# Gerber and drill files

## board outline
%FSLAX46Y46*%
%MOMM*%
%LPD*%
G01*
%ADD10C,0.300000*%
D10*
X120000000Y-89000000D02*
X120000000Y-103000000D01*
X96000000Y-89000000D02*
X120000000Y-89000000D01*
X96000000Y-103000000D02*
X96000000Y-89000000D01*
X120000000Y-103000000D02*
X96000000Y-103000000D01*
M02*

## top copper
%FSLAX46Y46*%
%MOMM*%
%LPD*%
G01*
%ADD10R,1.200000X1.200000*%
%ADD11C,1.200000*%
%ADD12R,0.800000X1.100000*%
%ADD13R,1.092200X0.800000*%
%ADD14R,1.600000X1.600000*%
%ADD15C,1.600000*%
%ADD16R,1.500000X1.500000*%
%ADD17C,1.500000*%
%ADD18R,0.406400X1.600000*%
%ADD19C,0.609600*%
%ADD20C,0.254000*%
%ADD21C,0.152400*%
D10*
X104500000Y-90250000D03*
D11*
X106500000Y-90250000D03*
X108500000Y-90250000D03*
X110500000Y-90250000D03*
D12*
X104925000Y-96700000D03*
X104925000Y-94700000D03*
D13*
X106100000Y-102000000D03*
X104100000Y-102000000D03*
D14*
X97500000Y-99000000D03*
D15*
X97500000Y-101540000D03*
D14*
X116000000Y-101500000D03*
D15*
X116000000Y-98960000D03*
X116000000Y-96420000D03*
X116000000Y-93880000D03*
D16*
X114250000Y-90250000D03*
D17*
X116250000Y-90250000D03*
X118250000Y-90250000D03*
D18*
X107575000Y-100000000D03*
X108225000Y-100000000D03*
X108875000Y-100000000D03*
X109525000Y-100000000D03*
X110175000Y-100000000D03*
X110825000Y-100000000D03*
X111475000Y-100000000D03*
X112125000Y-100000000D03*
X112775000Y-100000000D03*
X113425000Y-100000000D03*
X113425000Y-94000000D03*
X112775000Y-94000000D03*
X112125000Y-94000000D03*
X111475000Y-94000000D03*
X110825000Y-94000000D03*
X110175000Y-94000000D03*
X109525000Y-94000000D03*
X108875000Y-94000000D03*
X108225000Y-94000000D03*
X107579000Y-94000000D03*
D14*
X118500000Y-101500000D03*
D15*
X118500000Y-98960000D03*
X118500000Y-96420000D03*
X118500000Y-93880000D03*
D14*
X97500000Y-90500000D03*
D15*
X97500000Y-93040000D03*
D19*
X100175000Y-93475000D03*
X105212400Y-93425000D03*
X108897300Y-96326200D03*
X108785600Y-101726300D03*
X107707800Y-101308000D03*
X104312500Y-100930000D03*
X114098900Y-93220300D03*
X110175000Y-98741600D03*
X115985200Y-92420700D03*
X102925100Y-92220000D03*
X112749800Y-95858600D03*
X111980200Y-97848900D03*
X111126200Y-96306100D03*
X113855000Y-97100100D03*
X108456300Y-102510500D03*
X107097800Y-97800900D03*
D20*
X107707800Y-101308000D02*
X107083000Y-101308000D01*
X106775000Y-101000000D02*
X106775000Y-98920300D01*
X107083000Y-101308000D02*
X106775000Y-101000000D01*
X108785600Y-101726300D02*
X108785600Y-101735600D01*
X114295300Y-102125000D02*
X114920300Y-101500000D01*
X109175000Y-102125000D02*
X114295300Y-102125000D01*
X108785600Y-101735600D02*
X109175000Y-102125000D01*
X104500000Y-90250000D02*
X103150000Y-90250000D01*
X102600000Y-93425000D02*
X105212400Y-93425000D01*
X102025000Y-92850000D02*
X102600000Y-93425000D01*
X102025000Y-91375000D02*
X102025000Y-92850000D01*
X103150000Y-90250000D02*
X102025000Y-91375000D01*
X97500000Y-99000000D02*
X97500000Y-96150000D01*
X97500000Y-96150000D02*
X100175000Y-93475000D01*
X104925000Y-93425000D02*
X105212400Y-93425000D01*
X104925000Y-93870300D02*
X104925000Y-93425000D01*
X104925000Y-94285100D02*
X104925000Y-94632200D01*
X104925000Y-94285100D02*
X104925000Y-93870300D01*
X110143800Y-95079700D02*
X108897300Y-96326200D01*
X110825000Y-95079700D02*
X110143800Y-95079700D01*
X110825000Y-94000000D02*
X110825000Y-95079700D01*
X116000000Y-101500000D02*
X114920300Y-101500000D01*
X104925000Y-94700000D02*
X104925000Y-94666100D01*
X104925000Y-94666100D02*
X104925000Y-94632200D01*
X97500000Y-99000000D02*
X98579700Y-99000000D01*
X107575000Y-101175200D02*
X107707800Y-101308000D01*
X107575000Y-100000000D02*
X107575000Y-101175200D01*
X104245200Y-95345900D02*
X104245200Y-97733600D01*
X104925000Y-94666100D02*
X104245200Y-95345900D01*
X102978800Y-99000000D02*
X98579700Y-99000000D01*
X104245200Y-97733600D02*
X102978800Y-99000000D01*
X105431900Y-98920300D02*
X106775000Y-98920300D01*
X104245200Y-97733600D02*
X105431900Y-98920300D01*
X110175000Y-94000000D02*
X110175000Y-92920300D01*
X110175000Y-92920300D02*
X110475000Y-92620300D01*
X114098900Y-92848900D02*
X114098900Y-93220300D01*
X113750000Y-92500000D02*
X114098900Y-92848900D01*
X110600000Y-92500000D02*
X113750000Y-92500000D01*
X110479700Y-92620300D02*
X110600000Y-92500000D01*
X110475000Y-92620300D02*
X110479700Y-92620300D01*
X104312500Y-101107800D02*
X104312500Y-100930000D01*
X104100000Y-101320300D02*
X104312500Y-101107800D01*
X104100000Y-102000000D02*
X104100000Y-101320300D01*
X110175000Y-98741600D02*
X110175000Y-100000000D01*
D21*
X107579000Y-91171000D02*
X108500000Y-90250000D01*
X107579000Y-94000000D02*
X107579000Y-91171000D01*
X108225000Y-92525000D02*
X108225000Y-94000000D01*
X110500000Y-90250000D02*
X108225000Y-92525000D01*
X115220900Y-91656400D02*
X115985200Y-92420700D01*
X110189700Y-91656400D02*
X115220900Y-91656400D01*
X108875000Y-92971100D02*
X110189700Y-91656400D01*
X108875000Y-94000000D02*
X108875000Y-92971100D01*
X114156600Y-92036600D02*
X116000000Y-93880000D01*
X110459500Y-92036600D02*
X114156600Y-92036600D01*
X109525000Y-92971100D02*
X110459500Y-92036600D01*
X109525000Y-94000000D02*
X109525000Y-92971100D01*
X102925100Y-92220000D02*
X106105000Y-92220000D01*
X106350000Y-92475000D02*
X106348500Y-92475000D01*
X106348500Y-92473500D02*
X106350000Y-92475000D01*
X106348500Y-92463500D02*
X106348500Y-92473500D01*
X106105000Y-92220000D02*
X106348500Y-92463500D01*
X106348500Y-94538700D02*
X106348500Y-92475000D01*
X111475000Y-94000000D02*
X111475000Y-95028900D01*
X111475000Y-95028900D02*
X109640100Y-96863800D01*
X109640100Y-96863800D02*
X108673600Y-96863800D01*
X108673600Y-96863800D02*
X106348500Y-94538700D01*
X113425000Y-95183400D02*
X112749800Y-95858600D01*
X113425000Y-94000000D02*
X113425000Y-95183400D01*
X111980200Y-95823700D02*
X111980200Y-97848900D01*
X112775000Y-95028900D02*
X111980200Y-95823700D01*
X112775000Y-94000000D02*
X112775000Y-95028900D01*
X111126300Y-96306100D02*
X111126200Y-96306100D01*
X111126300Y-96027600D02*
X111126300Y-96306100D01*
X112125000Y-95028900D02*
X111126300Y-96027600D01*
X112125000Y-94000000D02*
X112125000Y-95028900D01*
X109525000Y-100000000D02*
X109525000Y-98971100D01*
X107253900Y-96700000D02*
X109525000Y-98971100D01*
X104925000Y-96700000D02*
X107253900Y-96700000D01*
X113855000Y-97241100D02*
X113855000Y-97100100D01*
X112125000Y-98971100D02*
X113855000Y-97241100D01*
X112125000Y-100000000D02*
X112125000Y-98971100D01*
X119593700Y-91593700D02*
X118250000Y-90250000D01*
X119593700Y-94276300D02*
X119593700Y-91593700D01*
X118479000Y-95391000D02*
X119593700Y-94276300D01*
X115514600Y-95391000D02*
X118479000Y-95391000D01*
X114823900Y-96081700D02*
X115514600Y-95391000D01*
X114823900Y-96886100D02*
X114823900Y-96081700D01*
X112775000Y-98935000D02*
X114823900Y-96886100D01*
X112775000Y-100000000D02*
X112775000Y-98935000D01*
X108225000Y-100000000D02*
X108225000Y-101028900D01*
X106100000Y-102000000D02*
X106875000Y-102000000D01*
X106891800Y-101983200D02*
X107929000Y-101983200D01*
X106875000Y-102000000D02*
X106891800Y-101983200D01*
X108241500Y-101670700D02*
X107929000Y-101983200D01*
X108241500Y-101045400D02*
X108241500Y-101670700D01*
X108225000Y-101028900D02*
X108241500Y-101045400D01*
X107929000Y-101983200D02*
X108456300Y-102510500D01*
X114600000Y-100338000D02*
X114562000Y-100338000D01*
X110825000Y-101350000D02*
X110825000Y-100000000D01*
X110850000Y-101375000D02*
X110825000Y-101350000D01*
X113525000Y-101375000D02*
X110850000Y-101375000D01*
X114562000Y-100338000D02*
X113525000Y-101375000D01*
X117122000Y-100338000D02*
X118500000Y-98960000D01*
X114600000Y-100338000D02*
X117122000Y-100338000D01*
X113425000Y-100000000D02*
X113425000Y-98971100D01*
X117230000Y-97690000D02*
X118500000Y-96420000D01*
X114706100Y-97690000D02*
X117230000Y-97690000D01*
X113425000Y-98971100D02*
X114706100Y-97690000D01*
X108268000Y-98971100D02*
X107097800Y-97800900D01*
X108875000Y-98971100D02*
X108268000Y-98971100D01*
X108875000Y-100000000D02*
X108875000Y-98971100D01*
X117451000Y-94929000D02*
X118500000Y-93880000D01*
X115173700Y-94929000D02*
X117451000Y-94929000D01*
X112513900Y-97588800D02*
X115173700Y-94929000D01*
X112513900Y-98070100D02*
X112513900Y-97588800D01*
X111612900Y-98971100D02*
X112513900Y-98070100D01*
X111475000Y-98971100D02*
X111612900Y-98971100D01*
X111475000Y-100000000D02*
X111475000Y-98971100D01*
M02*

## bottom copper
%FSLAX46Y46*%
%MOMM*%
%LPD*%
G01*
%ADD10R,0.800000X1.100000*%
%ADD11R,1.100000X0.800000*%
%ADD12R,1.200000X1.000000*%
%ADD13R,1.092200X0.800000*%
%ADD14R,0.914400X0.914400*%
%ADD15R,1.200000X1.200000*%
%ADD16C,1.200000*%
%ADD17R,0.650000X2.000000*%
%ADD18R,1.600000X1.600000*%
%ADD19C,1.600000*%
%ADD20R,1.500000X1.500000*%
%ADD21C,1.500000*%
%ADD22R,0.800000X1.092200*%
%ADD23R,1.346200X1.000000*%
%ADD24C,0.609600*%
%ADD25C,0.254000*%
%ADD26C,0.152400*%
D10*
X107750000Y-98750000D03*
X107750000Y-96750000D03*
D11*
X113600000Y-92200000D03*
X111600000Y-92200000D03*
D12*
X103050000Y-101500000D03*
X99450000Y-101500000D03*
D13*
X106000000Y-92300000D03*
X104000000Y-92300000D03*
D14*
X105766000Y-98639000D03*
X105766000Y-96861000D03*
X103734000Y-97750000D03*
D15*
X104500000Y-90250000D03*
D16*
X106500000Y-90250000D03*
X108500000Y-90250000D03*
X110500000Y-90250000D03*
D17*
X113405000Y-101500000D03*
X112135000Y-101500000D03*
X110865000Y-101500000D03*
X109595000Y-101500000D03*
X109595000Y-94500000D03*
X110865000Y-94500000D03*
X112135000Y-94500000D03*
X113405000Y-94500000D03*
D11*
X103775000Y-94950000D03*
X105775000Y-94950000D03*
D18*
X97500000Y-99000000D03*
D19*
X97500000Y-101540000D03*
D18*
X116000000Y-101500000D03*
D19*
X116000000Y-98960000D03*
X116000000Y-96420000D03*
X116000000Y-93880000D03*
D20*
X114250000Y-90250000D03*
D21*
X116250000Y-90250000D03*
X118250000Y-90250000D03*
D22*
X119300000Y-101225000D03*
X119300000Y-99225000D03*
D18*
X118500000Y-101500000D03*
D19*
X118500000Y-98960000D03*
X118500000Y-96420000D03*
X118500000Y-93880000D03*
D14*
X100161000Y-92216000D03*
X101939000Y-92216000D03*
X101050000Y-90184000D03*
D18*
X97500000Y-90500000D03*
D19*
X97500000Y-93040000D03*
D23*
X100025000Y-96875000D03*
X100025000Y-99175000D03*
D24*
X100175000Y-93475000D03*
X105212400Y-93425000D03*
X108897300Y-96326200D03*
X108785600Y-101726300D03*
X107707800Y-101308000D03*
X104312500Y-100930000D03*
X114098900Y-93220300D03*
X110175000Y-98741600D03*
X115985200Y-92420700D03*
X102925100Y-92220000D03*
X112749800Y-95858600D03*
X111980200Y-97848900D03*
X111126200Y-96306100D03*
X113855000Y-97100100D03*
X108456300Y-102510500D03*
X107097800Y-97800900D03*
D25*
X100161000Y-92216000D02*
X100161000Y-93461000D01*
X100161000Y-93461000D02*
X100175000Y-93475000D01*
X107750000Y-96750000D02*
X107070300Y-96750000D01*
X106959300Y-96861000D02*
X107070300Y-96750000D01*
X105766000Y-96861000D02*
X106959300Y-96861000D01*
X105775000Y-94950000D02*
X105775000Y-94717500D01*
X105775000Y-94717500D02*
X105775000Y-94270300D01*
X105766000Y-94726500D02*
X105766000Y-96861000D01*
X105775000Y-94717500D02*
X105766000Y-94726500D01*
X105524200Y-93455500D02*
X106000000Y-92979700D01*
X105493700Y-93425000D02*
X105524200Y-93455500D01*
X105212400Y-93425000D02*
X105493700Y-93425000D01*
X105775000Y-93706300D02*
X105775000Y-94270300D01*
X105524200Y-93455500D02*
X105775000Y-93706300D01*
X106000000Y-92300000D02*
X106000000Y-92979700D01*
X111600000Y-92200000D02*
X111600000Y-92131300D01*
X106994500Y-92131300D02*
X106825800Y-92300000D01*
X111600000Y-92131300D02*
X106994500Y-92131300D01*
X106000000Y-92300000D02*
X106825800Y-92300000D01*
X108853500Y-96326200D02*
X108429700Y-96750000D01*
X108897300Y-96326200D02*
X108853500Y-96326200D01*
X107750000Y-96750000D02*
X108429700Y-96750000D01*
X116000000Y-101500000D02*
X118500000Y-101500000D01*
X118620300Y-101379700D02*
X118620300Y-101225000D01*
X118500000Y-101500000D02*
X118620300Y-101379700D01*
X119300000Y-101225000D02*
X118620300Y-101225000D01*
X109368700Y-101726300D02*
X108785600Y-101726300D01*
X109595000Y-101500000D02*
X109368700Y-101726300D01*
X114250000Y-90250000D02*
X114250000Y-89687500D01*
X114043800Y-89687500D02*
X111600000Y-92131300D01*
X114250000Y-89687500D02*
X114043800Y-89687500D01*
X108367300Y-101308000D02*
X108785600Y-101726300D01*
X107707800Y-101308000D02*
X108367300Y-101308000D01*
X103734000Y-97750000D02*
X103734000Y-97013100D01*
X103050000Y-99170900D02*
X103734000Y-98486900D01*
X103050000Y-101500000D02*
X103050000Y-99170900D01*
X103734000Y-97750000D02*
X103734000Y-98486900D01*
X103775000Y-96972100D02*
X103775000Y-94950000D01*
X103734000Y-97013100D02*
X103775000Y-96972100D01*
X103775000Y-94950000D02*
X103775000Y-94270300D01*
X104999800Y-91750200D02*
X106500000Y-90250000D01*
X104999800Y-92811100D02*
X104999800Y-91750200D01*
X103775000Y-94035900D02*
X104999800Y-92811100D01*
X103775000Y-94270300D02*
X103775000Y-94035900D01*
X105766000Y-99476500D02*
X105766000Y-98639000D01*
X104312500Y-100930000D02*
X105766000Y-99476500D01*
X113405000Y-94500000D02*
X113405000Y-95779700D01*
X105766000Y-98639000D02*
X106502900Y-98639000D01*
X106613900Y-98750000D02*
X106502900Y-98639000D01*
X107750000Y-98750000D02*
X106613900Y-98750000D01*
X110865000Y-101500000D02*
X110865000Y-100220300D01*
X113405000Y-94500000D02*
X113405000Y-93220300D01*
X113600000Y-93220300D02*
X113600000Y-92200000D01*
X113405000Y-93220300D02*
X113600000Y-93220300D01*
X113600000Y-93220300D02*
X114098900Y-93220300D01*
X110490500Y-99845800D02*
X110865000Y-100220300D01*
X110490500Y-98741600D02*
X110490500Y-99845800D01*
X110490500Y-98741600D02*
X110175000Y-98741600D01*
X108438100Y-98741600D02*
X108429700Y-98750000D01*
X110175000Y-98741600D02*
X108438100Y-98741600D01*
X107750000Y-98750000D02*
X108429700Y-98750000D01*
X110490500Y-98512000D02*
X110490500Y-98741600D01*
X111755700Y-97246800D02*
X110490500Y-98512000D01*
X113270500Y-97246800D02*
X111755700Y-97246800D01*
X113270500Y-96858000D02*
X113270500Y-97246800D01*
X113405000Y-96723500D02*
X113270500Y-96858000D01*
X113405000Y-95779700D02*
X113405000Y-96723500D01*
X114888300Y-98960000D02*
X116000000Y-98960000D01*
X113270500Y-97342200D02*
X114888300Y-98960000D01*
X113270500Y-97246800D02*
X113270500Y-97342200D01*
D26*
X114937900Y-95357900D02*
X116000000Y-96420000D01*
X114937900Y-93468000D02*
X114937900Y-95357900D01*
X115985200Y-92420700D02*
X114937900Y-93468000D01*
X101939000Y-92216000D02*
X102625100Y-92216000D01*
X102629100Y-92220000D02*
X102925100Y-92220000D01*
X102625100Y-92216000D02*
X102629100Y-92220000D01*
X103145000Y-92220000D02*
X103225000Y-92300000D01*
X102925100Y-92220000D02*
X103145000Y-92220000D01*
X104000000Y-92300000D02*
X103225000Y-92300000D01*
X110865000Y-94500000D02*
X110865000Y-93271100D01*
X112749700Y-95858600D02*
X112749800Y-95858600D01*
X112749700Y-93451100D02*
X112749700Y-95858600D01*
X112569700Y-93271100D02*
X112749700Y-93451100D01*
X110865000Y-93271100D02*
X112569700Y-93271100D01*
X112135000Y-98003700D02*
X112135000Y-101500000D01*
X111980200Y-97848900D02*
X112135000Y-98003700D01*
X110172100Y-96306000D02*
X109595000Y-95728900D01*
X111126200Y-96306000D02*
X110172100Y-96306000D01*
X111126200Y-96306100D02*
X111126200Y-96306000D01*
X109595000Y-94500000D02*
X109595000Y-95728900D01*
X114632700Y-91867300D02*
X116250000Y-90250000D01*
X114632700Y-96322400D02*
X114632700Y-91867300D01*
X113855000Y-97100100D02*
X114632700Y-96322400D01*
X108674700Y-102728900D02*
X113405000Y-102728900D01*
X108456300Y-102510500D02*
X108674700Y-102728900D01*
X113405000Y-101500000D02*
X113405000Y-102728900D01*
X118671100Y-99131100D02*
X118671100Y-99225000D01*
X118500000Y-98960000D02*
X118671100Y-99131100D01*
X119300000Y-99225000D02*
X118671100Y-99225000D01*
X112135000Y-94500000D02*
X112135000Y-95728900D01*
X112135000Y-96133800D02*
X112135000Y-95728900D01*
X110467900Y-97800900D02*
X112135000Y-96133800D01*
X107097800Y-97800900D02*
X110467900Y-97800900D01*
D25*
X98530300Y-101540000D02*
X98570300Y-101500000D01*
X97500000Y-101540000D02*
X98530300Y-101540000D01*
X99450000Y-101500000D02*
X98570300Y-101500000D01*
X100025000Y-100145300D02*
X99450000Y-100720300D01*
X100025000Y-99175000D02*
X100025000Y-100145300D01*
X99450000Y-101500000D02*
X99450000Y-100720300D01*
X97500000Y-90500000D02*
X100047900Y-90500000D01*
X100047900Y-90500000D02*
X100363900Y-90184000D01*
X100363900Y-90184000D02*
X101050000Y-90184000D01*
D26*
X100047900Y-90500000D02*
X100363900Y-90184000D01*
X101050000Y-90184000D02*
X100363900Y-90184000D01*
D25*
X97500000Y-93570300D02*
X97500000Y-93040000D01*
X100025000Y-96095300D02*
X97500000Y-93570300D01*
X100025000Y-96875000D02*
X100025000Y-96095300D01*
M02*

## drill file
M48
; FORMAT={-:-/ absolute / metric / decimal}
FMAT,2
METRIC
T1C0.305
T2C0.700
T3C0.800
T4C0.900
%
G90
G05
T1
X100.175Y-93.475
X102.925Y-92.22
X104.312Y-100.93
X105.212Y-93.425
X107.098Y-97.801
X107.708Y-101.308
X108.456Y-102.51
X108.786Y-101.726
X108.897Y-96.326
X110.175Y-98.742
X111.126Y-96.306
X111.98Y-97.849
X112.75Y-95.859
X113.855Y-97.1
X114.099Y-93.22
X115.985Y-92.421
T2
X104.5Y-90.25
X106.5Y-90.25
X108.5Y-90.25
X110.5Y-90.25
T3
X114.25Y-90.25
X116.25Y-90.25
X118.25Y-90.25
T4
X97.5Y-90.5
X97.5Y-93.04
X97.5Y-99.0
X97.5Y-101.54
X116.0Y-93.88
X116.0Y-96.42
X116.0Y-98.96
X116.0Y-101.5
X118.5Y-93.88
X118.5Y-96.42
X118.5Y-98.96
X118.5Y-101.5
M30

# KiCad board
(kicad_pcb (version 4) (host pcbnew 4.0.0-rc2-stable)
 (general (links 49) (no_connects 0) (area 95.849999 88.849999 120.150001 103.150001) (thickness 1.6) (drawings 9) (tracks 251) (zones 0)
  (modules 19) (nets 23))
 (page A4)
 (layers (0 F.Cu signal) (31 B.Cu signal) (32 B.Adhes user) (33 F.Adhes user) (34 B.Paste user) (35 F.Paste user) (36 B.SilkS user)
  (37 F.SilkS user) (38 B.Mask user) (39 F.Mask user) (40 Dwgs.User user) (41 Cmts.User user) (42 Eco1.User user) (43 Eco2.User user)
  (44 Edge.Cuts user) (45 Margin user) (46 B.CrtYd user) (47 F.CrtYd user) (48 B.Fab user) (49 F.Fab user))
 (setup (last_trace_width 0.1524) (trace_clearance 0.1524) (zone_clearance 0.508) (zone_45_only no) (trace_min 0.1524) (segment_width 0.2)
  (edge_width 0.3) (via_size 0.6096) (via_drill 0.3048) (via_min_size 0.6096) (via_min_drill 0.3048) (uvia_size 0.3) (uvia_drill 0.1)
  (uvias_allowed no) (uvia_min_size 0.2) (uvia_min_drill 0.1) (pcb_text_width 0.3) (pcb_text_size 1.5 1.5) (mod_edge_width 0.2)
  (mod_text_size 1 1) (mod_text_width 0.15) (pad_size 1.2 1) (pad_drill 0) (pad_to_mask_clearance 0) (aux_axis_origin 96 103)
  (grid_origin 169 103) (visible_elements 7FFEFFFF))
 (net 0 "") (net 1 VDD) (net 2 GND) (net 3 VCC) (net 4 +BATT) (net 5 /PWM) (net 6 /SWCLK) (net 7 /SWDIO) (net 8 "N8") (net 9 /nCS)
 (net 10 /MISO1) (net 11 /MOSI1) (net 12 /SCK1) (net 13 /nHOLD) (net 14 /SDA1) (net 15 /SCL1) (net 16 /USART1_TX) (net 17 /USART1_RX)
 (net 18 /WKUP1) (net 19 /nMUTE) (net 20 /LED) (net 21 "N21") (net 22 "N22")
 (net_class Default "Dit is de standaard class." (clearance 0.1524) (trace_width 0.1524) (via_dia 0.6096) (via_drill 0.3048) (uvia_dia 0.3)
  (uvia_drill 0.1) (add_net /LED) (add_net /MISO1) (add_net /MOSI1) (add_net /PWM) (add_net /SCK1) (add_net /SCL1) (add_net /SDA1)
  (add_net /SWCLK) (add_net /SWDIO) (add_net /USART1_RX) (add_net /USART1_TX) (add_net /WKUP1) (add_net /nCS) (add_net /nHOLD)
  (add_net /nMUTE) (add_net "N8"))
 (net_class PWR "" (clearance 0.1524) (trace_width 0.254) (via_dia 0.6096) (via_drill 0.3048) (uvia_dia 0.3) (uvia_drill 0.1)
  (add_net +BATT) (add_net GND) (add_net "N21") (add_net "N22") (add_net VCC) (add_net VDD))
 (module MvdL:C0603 (layer B.Cu) (at 107.75 97.75 90)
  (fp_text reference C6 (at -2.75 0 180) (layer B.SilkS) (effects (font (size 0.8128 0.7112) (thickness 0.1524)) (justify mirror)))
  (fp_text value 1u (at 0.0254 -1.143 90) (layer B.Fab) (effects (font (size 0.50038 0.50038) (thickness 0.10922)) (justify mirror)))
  (pad 1 smd rect (at -1 0 90) (size 1.1 0.8) (layers B.Cu B.Paste B.Mask) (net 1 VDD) (clearance 0.1524))
  (pad 2 smd rect (at 1 0 90) (size 1.1 0.8) (layers B.Cu B.Paste B.Mask) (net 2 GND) (clearance 0.1524)))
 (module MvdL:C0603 (layer B.Cu) (at 112.6 92.2 180)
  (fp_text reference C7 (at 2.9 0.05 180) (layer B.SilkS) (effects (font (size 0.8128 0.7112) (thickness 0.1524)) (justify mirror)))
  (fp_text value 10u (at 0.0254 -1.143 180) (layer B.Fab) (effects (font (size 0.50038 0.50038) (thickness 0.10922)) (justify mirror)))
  (pad 1 smd rect (at -1 0 180) (size 1.1 0.8) (layers B.Cu B.Paste B.Mask) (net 1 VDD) (clearance 0.1524))
  (pad 2 smd rect (at 1 0 180) (size 1.1 0.8) (layers B.Cu B.Paste B.Mask) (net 2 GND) (clearance 0.1524)))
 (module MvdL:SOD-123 (layer B.Cu) (at 101.25 101.5 180)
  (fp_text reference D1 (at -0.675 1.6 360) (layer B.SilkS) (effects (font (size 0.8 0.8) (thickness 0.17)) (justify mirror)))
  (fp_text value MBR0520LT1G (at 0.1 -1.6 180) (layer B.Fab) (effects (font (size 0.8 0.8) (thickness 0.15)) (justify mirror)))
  (pad K smd rect (at -1.8 0 180) (size 1.2 1) (layers B.Cu B.Paste B.Mask) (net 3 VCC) (clearance 0.1524))
  (pad A smd rect (at 1.8 0 180) (size 1.2 1) (layers B.Cu B.Paste B.Mask) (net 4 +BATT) (clearance 0.1524)))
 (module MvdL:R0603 (layer B.Cu) (at 105 92.3 180)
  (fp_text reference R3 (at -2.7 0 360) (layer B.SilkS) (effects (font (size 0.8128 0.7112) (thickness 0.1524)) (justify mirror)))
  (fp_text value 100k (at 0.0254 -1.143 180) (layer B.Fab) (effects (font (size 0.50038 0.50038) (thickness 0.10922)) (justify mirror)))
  (pad 1 smd rect (at -1 0 180) (size 1.0922 0.8) (layers B.Cu B.Paste B.Mask) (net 2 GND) (clearance 0.1524))
  (pad 2 smd rect (at 1 0 180) (size 1.0922 0.8) (layers B.Cu B.Paste B.Mask) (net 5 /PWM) (clearance 0.1524)))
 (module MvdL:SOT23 (layer B.Cu) (at 104.75 97.75 90)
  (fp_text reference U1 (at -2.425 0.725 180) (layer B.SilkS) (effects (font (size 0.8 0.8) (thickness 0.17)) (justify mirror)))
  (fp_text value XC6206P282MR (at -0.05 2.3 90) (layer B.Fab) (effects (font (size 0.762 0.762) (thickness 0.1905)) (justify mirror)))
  (pad 2 smd rect (at -0.889 1.016 90) (size 0.9144 0.9144) (layers B.Cu B.Paste B.Mask) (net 1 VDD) (die_length -2147.483648)
   (clearance 0.1524))
  (pad 1 smd rect (at 0.889 1.016 90) (size 0.9144 0.9144) (layers B.Cu B.Paste B.Mask) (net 2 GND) (clearance 0.1524))
  (pad 3 smd rect (at 0 -1.016 90) (size 0.9144 0.9144) (layers B.Cu B.Paste B.Mask) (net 3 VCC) (clearance 0.1524)))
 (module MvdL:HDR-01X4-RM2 (layer F.Cu) (at 104.5 90.25)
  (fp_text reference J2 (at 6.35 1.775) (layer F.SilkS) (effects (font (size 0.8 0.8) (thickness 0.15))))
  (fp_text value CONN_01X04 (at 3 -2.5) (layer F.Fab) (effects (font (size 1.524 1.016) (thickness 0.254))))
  (pad 1 thru_hole rect (at 0 0) (size 1.2 1.2) (drill 0.7) (layers *.Cu *.Mask F.SilkS) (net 2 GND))
  (pad 2 thru_hole circle (at 2 0) (size 1.2 1.2) (drill 0.7) (layers *.Cu *.Mask F.SilkS) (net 3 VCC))
  (pad 3 thru_hole circle (at 4 0) (size 1.2 1.2) (drill 0.7) (layers *.Cu *.Mask F.SilkS) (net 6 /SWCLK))
  (pad 4 thru_hole circle (at 6 0) (size 1.2 1.2) (drill 0.7) (layers *.Cu *.Mask F.SilkS) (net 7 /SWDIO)))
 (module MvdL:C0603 (layer F.Cu) (at 104.925 95.7 90)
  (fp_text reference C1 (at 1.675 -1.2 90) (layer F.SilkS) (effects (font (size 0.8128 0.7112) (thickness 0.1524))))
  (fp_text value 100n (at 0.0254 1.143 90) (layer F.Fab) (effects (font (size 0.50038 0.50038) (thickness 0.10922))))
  (pad 1 smd rect (at -1 0 90) (size 1.1 0.8) (layers F.Cu F.Paste F.Mask) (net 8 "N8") (clearance 0.1524))
  (pad 2 smd rect (at 1 0 90) (size 1.1 0.8) (layers F.Cu F.Paste F.Mask) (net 2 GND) (clearance 0.1524)))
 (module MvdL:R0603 (layer F.Cu) (at 105.1 102 180)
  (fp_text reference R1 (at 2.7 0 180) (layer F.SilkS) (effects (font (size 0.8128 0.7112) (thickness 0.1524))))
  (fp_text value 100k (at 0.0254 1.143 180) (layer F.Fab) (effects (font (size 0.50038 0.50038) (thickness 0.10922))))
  (pad 1 smd rect (at -1 0 180) (size 1.0922 0.8) (layers F.Cu F.Paste F.Mask) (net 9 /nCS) (clearance 0.1524))
  (pad 2 smd rect (at 1 0 180) (size 1.0922 0.8) (layers F.Cu F.Paste F.Mask) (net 1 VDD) (clearance 0.1524)))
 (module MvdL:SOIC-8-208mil (layer B.Cu) (at 111.5 98 90)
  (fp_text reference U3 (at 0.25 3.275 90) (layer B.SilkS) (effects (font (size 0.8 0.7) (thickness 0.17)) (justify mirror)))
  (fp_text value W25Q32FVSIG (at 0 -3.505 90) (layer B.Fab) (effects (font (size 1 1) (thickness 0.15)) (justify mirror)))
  (pad 1 smd rect (at -3.5 1.905 90) (size 2 0.65) (layers B.Cu B.Paste B.Mask) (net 9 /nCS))
  (pad 2 smd rect (at -3.5 0.635 90) (size 2 0.65) (layers B.Cu B.Paste B.Mask) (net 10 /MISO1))
  (pad 3 smd rect (at -3.5 -0.635 90) (size 2 0.65) (layers B.Cu B.Paste B.Mask) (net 1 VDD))
  (pad 4 smd rect (at -3.5 -1.905 90) (size 2 0.65) (layers B.Cu B.Paste B.Mask) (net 2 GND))
  (pad 5 smd rect (at 3.5 -1.905 90) (size 2 0.65) (layers B.Cu B.Paste B.Mask) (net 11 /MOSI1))
  (pad 6 smd rect (at 3.5 -0.635 90) (size 2 0.65) (layers B.Cu B.Paste B.Mask) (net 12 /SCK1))
  (pad 7 smd rect (at 3.5 0.635 90) (size 2 0.65) (layers B.Cu B.Paste B.Mask) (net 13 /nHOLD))
  (pad 8 smd rect (at 3.5 1.905 90) (size 2 0.65) (layers B.Cu B.Paste B.Mask) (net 1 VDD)))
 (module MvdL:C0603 (layer B.Cu) (at 104.775 94.95)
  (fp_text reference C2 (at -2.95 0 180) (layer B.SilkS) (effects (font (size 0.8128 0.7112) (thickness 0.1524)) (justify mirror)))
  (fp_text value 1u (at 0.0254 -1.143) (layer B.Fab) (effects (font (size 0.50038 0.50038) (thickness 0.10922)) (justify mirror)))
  (pad 1 smd rect (at -1 0) (size 1.1 0.8) (layers B.Cu B.Paste B.Mask) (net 3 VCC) (clearance 0.1524))
  (pad 2 smd rect (at 1 0) (size 1.1 0.8) (layers B.Cu B.Paste B.Mask) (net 2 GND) (clearance 0.1524)))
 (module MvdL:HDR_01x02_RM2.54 (layer F.Cu) (at 97.5 99 270)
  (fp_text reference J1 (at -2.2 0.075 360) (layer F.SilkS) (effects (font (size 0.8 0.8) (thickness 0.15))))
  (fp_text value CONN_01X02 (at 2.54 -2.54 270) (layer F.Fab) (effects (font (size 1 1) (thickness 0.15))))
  (pad 1 thru_hole rect (at 0 0 270) (size 1.6 1.6) (drill 0.9) (layers *.Cu *.Mask F.SilkS) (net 2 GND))
  (pad 2 thru_hole circle (at 2.54 0 270) (size 1.6 1.6) (drill 0.9) (layers *.Cu *.Mask F.SilkS) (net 4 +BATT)))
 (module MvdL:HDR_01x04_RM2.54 (layer F.Cu) (at 116 101.5 90)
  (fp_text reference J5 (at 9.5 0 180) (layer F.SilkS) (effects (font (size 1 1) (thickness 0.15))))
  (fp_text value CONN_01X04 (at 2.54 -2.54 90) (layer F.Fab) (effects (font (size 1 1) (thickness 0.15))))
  (pad 1 thru_hole rect (at 0 0 90) (size 1.6 1.6) (drill 0.9) (layers *.Cu *.Mask F.SilkS) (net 2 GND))
  (pad 2 thru_hole circle (at 2.54 0 90) (size 1.6 1.6) (drill 0.9) (layers *.Cu *.Mask F.SilkS) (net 1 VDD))
  (pad 3 thru_hole circle (at 5.08 0 90) (size 1.6 1.6) (drill 0.9) (layers *.Cu *.Mask F.SilkS) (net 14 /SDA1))
  (pad 4 thru_hole circle (at 7.62 0 90) (size 1.6 1.6) (drill 0.9) (layers *.Cu *.Mask F.SilkS) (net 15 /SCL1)))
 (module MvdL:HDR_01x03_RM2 (layer F.Cu) (at 114.25 90.25)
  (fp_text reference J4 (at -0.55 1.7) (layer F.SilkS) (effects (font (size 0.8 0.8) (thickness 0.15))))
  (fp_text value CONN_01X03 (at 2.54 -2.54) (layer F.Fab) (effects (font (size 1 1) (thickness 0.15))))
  (pad 1 thru_hole rect (at 0 0) (size 1.5 1.5) (drill 0.8) (layers *.Cu *.Mask F.SilkS) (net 2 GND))
  (pad 2 thru_hole circle (at 2 0) (size 1.5 1.5) (drill 0.8) (layers *.Cu *.Mask F.SilkS) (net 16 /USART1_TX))
  (pad 3 thru_hole circle (at 4 0) (size 1.5 1.5) (drill 0.8) (layers *.Cu *.Mask F.SilkS) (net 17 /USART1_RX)))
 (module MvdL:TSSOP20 (layer F.Cu) (at 110.5 97)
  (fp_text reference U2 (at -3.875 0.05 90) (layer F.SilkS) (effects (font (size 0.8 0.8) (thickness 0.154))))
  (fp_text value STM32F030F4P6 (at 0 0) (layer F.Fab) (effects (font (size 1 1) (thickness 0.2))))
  (pad 1 smd rect (at -2.925 3) (size 0.4064 1.6) (layers F.Cu F.Paste F.Mask) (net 2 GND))
  (pad 2 smd rect (at -2.275 3) (size 0.4064 1.6) (layers F.Cu F.Paste F.Mask) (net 9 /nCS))
  (pad 3 smd rect (at -1.625 3) (size 0.4064 1.6) (layers F.Cu F.Paste F.Mask) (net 13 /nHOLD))
  (pad 4 smd rect (at -0.975 3) (size 0.4064 1.6) (layers F.Cu F.Paste F.Mask) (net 8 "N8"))
  (pad 5 smd rect (at -0.325 3) (size 0.4064 1.6) (layers F.Cu F.Paste F.Mask) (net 1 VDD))
  (pad 6 smd rect (at 0.325 3) (size 0.4064 1.6) (layers F.Cu F.Paste F.Mask) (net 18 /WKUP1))
  (pad 7 smd rect (at 0.975 3) (size 0.4064 1.6) (layers F.Cu F.Paste F.Mask) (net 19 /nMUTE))
  (pad 8 smd rect (at 1.625 3) (size 0.4064 1.6) (layers F.Cu F.Paste F.Mask) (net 16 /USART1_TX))
  (pad 9 smd rect (at 2.275 3) (size 0.4064 1.6) (layers F.Cu F.Paste F.Mask) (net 17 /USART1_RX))
  (pad 10 smd rect (at 2.925 3) (size 0.4064 1.6) (layers F.Cu F.Paste F.Mask) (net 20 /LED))
  (pad 11 smd rect (at 2.925 -3) (size 0.4064 1.6) (layers F.Cu F.Paste F.Mask) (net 12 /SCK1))
  (pad 12 smd rect (at 2.275 -3) (size 0.4064 1.6) (layers F.Cu F.Paste F.Mask) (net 10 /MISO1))
  (pad 13 smd rect (at 1.625 -3) (size 0.4064 1.6) (layers F.Cu F.Paste F.Mask) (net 11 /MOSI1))
  (pad 14 smd rect (at 0.975 -3) (size 0.4064 1.6) (layers F.Cu F.Paste F.Mask) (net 5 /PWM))
  (pad 15 smd rect (at 0.325 -3) (size 0.4064 1.6) (layers F.Cu F.Paste F.Mask) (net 2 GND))
  (pad 16 smd rect (at -0.325 -3) (size 0.4064 1.6) (layers F.Cu F.Paste F.Mask) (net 1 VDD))
  (pad 17 smd rect (at -0.975 -3) (size 0.4064 1.6) (layers F.Cu F.Paste F.Mask) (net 15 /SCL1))
  (pad 18 smd rect (at -1.625 -3) (size 0.4064 1.6) (layers F.Cu F.Paste F.Mask) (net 14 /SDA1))
  (pad 19 smd rect (at -2.275 -3) (size 0.4064 1.6) (layers F.Cu F.Paste F.Mask) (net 7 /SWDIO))
  (pad 20 smd rect (at -2.921 -3) (size 0.4064 1.6) (layers F.Cu F.Paste F.Mask) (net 6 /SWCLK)))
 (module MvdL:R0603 (layer B.Cu) (at 119.3 100.225 90)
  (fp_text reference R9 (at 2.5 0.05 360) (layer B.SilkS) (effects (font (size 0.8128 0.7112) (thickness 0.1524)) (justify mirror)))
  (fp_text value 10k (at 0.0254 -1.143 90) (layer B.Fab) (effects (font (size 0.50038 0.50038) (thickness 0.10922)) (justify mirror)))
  (pad 1 smd rect (at -1 0 90) (size 1.0922 0.8) (layers B.Cu B.Paste B.Mask) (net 2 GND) (clearance 0.1524))
  (pad 2 smd rect (at 1 0 90) (size 1.0922 0.8) (layers B.Cu B.Paste B.Mask) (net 18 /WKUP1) (clearance 0.1524)))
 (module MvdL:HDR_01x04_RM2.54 (layer F.Cu) (at 118.5 101.5 90)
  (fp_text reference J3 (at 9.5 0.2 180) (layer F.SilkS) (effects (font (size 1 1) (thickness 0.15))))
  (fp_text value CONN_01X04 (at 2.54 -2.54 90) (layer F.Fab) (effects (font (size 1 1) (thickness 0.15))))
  (pad 1 thru_hole rect (at 0 0 90) (size 1.6 1.6) (drill 0.9) (layers *.Cu *.Mask F.SilkS) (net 2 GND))
  (pad 2 thru_hole circle (at 2.54 0 90) (size 1.6 1.6) (drill 0.9) (layers *.Cu *.Mask F.SilkS) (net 18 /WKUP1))
  (pad 3 thru_hole circle (at 5.08 0 90) (size 1.6 1.6) (drill 0.9) (layers *.Cu *.Mask F.SilkS) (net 20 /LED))
  (pad 4 thru_hole circle (at 7.62 0 90) (size 1.6 1.6) (drill 0.9) (layers *.Cu *.Mask F.SilkS) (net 19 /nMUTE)))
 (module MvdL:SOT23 (layer B.Cu) (at 101.05 91.2)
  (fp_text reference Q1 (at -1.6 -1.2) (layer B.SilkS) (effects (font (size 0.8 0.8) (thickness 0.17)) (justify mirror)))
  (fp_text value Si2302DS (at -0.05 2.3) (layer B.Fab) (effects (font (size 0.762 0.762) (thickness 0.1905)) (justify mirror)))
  (pad 2 smd rect (at -0.889 1.016) (size 0.9144 0.9144) (layers B.Cu B.Paste B.Mask) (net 2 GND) (die_length -2147.483648)
   (clearance 0.1524))
  (pad 1 smd rect (at 0.889 1.016) (size 0.9144 0.9144) (layers B.Cu B.Paste B.Mask) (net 5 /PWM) (clearance 0.1524))
  (pad 3 smd rect (at 0 -1.016) (size 0.9144 0.9144) (layers B.Cu B.Paste B.Mask) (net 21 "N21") (clearance 0.1524)))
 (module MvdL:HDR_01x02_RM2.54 (layer F.Cu) (at 97.5 90.5 270)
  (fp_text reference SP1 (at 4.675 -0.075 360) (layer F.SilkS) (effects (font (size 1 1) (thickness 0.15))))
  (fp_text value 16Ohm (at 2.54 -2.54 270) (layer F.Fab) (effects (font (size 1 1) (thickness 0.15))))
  (pad 1 thru_hole rect (at 0 0 270) (size 1.6 1.6) (drill 0.9) (layers *.Cu *.Mask F.SilkS) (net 21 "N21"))
  (pad 2 thru_hole circle (at 2.54 0 270) (size 1.6 1.6) (drill 0.9) (layers *.Cu *.Mask F.SilkS) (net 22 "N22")))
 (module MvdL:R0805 (layer B.Cu) (at 100.025 98.025 270)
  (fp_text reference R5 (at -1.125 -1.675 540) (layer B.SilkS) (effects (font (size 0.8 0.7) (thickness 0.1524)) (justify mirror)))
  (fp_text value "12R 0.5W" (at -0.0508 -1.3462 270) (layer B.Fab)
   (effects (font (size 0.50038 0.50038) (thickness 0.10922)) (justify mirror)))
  (pad 1 smd rect (at -1.15 0 270) (size 1 1.3462) (layers B.Cu B.Paste B.Mask) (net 22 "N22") (clearance 0.1524))
  (pad 2 smd rect (at 1.15 0 270) (size 1 1.3462) (layers B.Cu B.Paste B.Mask) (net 4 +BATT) (clearance 0.1524)))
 (gr_line (start 120 89) (end 120 103) (angle 90) (layer Edge.Cuts) (width 0.3))
 (gr_line (start 96 89) (end 120 89) (angle 90) (layer Edge.Cuts) (width 0.3))
 (gr_line (start 96 103) (end 96 89) (angle 90) (layer Edge.Cuts) (width 0.3))
 (gr_line (start 120 103) (end 96 103) (angle 90) (layer Edge.Cuts) (width 0.3))
 (segment (start 107.7078 101.308) (end 107.083 101.308) (width 0.254) (layer F.Cu) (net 2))
 (segment (start 106.775 101) (end 106.775 98.9203) (width 0.254) (layer F.Cu) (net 2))
 (segment (start 107.083 101.308) (end 106.775 101) (width 0.254) (layer F.Cu) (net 2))
 (segment (start 108.7856 101.7263) (end 108.7856 101.7356) (width 0.254) (layer F.Cu) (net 2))
 (segment (start 114.2953 102.125) (end 114.9203 101.5) (width 0.254) (layer F.Cu) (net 2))
 (segment (start 109.175 102.125) (end 114.2953 102.125) (width 0.254) (layer F.Cu) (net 2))
 (segment (start 108.7856 101.7356) (end 109.175 102.125) (width 0.254) (layer F.Cu) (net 2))
 (segment (start 104.5 90.25) (end 103.15 90.25) (width 0.254) (layer F.Cu) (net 2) (status 400000))
 (segment (start 102.6 93.425) (end 105.2124 93.425) (width 0.254) (layer F.Cu) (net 2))
 (segment (start 102.025 92.85) (end 102.6 93.425) (width 0.254) (layer F.Cu) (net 2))
 (segment (start 102.025 91.375) (end 102.025 92.85) (width 0.254) (layer F.Cu) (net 2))
 (segment (start 103.15 90.25) (end 102.025 91.375) (width 0.254) (layer F.Cu) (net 2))
 (segment (start 97.5 99) (end 97.5 96.15) (width 0.254) (layer F.Cu) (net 2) (status 400000))
 (segment (start 97.5 96.15) (end 100.175 93.475) (width 0.254) (layer F.Cu) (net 2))
 (segment (start 100.161 92.216) (end 100.161 93.461) (width 0.254) (layer B.Cu) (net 2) (status 400000))
 (segment (start 100.161 93.461) (end 100.175 93.475) (width 0.254) (layer B.Cu) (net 2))
 (via (at 100.175 93.475) (size 0.6096) (drill 0.3048) (layers F.Cu B.Cu) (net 2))
 (via (at 105.2124 93.425) (size 0.6096) (layers F.Cu B.Cu) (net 2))
 (via (at 108.8973 96.3262) (size 0.6096) (layers F.Cu B.Cu) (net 2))
 (via (at 108.7856 101.7263) (size 0.6096) (layers F.Cu B.Cu) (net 2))
 (via (at 107.7078 101.308) (size 0.6096) (layers F.Cu B.Cu) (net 2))
 (segment (start 107.75 96.75) (end 107.0703 96.75) (width 0.254) (layer B.Cu) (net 2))
 (segment (start 106.9593 96.861) (end 107.0703 96.75) (width 0.254) (layer B.Cu) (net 2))
 (segment (start 105.766 96.861) (end 106.9593 96.861) (width 0.254) (layer B.Cu) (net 2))
 (segment (start 105.775 94.95) (end 105.775 94.7175) (width 0.254) (layer B.Cu) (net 2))
 (segment (start 105.775 94.7175) (end 105.775 94.2703) (width 0.254) (layer B.Cu) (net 2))
 (segment (start 105.766 94.7265) (end 105.766 96.861) (width 0.254) (layer B.Cu) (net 2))
 (segment (start 105.775 94.7175) (end 105.766 94.7265) (width 0.254) (layer B.Cu) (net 2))
 (segment (start 104.925 93.425) (end 105.2124 93.425) (width 0.254) (layer F.Cu) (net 2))
 (segment (start 104.925 93.8703) (end 104.925 93.425) (width 0.254) (layer F.Cu) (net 2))
 (segment (start 105.5242 93.4555) (end 106 92.9797) (width 0.254) (layer B.Cu) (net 2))
 (segment (start 105.4937 93.425) (end 105.5242 93.4555) (width 0.254) (layer B.Cu) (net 2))
 (segment (start 105.2124 93.425) (end 105.4937 93.425) (width 0.254) (layer B.Cu) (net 2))
 (segment (start 105.775 93.7063) (end 105.775 94.2703) (width 0.254) (layer B.Cu) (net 2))
 (segment (start 105.5242 93.4555) (end 105.775 93.7063) (width 0.254) (layer B.Cu) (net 2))
 (segment (start 104.925 94.2851) (end 104.925 94.6322) (width 0.254) (layer F.Cu) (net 2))
 (segment (start 104.925 94.2851) (end 104.925 93.8703) (width 0.254) (layer F.Cu) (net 2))
 (segment (start 106 92.3) (end 106 92.9797) (width 0.254) (layer B.Cu) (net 2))
 (segment (start 111.6 92.2) (end 111.6 92.1313) (width 0.254) (layer B.Cu) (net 2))
 (segment (start 106.9945 92.1313) (end 106.8258 92.3) (width 0.254) (layer B.Cu) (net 2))
 (segment (start 111.6 92.1313) (end 106.9945 92.1313) (width 0.254) (layer B.Cu) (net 2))
 (segment (start 106 92.3) (end 106.8258 92.3) (width 0.254) (layer B.Cu) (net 2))
 (segment (start 110.1438 95.0797) (end 108.8973 96.3262) (width 0.254) (layer F.Cu) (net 2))
 (segment (start 110.825 95.0797) (end 110.1438 95.0797) (width 0.254) (layer F.Cu) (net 2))
 (segment (start 108.8535 96.3262) (end 108.4297 96.75) (width 0.254) (layer B.Cu) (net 2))
 (segment (start 108.8973 96.3262) (end 108.8535 96.3262) (width 0.254) (layer B.Cu) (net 2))
 (segment (start 110.825 94) (end 110.825 95.0797) (width 0.254) (layer F.Cu) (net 2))
 (segment (start 107.75 96.75) (end 108.4297 96.75) (width 0.254) (layer B.Cu) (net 2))
 (segment (start 116 101.5) (end 118.5 101.5) (width 0.254) (layer B.Cu) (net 2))
 (segment (start 118.6203 101.3797) (end 118.6203 101.225) (width 0.254) (layer B.Cu) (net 2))
 (segment (start 118.5 101.5) (end 118.6203 101.3797) (width 0.254) (layer B.Cu) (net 2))
 (segment (start 119.3 101.225) (end 118.6203 101.225) (width 0.254) (layer B.Cu) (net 2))
 (segment (start 109.3687 101.7263) (end 108.7856 101.7263) (width 0.254) (layer B.Cu) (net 2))
 (segment (start 109.595 101.5) (end 109.3687 101.7263) (width 0.254) (layer B.Cu) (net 2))
 (segment (start 116 101.5) (end 114.9203 101.5) (width 0.254) (layer F.Cu) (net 2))
 (segment (start 114.25 90.25) (end 114.25 89.6875) (width 0.254) (layer B.Cu) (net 2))
 (segment (start 114.0438 89.6875) (end 111.6 92.1313) (width 0.254) (layer B.Cu) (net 2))
 (segment (start 114.25 89.6875) (end 114.0438 89.6875) (width 0.254) (layer B.Cu) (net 2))
 (segment (start 104.925 94.7) (end 104.925 94.6661) (width 0.254) (layer F.Cu) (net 2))
 (segment (start 104.925 94.6661) (end 104.925 94.6322) (width 0.254) (layer F.Cu) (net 2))
 (segment (start 97.5 99) (end 98.5797 99) (width 0.254) (layer F.Cu) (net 2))
 (segment (start 107.575 101.1752) (end 107.7078 101.308) (width 0.254) (layer F.Cu) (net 2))
 (segment (start 107.575 100) (end 107.575 101.1752) (width 0.254) (layer F.Cu) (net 2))
 (segment (start 108.3673 101.308) (end 108.7856 101.7263) (width 0.254) (layer B.Cu) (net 2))
 (segment (start 107.7078 101.308) (end 108.3673 101.308) (width 0.254) (layer B.Cu) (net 2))
 (segment (start 104.2452 95.3459) (end 104.2452 97.7336) (width 0.254) (layer F.Cu) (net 2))
 (segment (start 104.925 94.6661) (end 104.2452 95.3459) (width 0.254) (layer F.Cu) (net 2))
 (segment (start 102.9788 99) (end 98.5797 99) (width 0.254) (layer F.Cu) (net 2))
 (segment (start 104.2452 97.7336) (end 102.9788 99) (width 0.254) (layer F.Cu) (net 2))
 (segment (start 105.4319 98.9203) (end 106.775 98.9203) (width 0.254) (layer F.Cu) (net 2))
 (segment (start 104.2452 97.7336) (end 105.4319 98.9203) (width 0.254) (layer F.Cu) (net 2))
 (segment (start 103.734 97.75) (end 103.734 97.0131) (width 0.254) (layer B.Cu) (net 3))
 (segment (start 103.05 99.1709) (end 103.734 98.4869) (width 0.254) (layer B.Cu) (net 3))
 (segment (start 103.05 101.5) (end 103.05 99.1709) (width 0.254) (layer B.Cu) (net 3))
 (segment (start 103.734 97.75) (end 103.734 98.4869) (width 0.254) (layer B.Cu) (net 3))
 (segment (start 103.775 96.9721) (end 103.775 94.95) (width 0.254) (layer B.Cu) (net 3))
 (segment (start 103.734 97.0131) (end 103.775 96.9721) (width 0.254) (layer B.Cu) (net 3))
 (segment (start 103.775 94.95) (end 103.775 94.2703) (width 0.254) (layer B.Cu) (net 3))
 (segment (start 104.9998 91.7502) (end 106.5 90.25) (width 0.254) (layer B.Cu) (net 3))
 (segment (start 104.9998 92.8111) (end 104.9998 91.7502) (width 0.254) (layer B.Cu) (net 3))
 (segment (start 103.775 94.0359) (end 104.9998 92.8111) (width 0.254) (layer B.Cu) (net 3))
 (segment (start 103.775 94.2703) (end 103.775 94.0359) (width 0.254) (layer B.Cu) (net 3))
 (segment (start 110.175 94) (end 110.175 92.9203) (width 0.254) (layer F.Cu) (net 1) (status 400000))
 (segment (start 110.175 92.9203) (end 110.475 92.6203) (width 0.254) (layer F.Cu) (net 1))
 (segment (start 114.0989 92.8489) (end 114.0989 93.2203) (width 0.254) (layer F.Cu) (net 1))
 (segment (start 113.75 92.5) (end 114.0989 92.8489) (width 0.254) (layer F.Cu) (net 1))
 (segment (start 110.6 92.5) (end 113.75 92.5) (width 0.254) (layer F.Cu) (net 1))
 (segment (start 110.4797 92.6203) (end 110.6 92.5) (width 0.254) (layer F.Cu) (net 1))
 (segment (start 110.475 92.6203) (end 110.4797 92.6203) (width 0.254) (layer F.Cu) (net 1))
 (via (at 104.3125 100.93) (size 0.6096) (layers F.Cu B.Cu) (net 1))
 (via (at 114.0989 93.2203) (size 0.6096) (layers F.Cu B.Cu) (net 1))
 (via (at 110.175 98.7416) (size 0.6096) (layers F.Cu B.Cu) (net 1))
 (segment (start 104.3125 101.1078) (end 104.3125 100.93) (width 0.254) (layer F.Cu) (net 1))
 (segment (start 104.1 101.3203) (end 104.3125 101.1078) (width 0.254) (layer F.Cu) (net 1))
 (segment (start 105.766 99.4765) (end 105.766 98.639) (width 0.254) (layer B.Cu) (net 1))
 (segment (start 104.3125 100.93) (end 105.766 99.4765) (width 0.254) (layer B.Cu) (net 1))
 (segment (start 104.1 102) (end 104.1 101.3203) (width 0.254) (layer F.Cu) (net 1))
 (segment (start 113.405 94.5) (end 113.405 95.7797) (width 0.254) (layer B.Cu) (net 1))
 (segment (start 105.766 98.639) (end 106.5029 98.639) (width 0.254) (layer B.Cu) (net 1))
 (segment (start 106.6139 98.75) (end 106.5029 98.639) (width 0.254) (layer B.Cu) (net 1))
 (segment (start 107.75 98.75) (end 106.6139 98.75) (width 0.254) (layer B.Cu) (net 1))
 (segment (start 110.865 101.5) (end 110.865 100.2203) (width 0.254) (layer B.Cu) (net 1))
 (segment (start 113.405 94.5) (end 113.405 93.2203) (width 0.254) (layer B.Cu) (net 1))
 (segment (start 113.6 93.2203) (end 113.6 92.2) (width 0.254) (layer B.Cu) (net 1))
 (segment (start 113.405 93.2203) (end 113.6 93.2203) (width 0.254) (layer B.Cu) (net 1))
 (segment (start 113.6 93.2203) (end 114.0989 93.2203) (width 0.254) (layer B.Cu) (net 1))
 (segment (start 110.175 98.7416) (end 110.175 100) (width 0.254) (layer F.Cu) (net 1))
 (segment (start 110.4905 99.8458) (end 110.865 100.2203) (width 0.254) (layer B.Cu) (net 1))
 (segment (start 110.4905 98.7416) (end 110.4905 99.8458) (width 0.254) (layer B.Cu) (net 1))
 (segment (start 110.4905 98.7416) (end 110.175 98.7416) (width 0.254) (layer B.Cu) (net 1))
 (segment (start 108.4381 98.7416) (end 108.4297 98.75) (width 0.254) (layer B.Cu) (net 1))
 (segment (start 110.175 98.7416) (end 108.4381 98.7416) (width 0.254) (layer B.Cu) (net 1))
 (segment (start 107.75 98.75) (end 108.4297 98.75) (width 0.254) (layer B.Cu) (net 1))
 (segment (start 110.4905 98.512) (end 110.4905 98.7416) (width 0.254) (layer B.Cu) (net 1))
 (segment (start 111.7557 97.2468) (end 110.4905 98.512) (width 0.254) (layer B.Cu) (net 1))
 (segment (start 113.2705 97.2468) (end 111.7557 97.2468) (width 0.254) (layer B.Cu) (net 1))
 (segment (start 113.2705 96.858) (end 113.2705 97.2468) (width 0.254) (layer B.Cu) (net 1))
 (segment (start 113.405 96.7235) (end 113.2705 96.858) (width 0.254) (layer B.Cu) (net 1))
 (segment (start 113.405 95.7797) (end 113.405 96.7235) (width 0.254) (layer B.Cu) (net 1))
 (segment (start 114.8883 98.96) (end 116 98.96) (width 0.254) (layer B.Cu) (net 1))
 (segment (start 113.2705 97.3422) (end 114.8883 98.96) (width 0.254) (layer B.Cu) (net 1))
 (segment (start 113.2705 97.2468) (end 113.2705 97.3422) (width 0.254) (layer B.Cu) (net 1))
 (segment (start 107.579 91.171) (end 108.5 90.25) (width 0.1524) (layer F.Cu) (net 6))
 (segment (start 107.579 94) (end 107.579 91.171) (width 0.1524) (layer F.Cu) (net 6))
 (segment (start 108.225 92.525) (end 108.225 94) (width 0.1524) (layer F.Cu) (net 7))
 (segment (start 110.5 90.25) (end 108.225 92.525) (width 0.1524) (layer F.Cu) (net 7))
 (via (at 115.9852 92.4207) (size 0.6096) (layers F.Cu B.Cu) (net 14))
 (segment (start 115.2209 91.6564) (end 115.9852 92.4207) (width 0.1524) (layer F.Cu) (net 14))
 (segment (start 110.1897 91.6564) (end 115.2209 91.6564) (width 0.1524) (layer F.Cu) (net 14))
 (segment (start 108.875 92.9711) (end 110.1897 91.6564) (width 0.1524) (layer F.Cu) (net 14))
 (segment (start 114.9379 95.3579) (end 116 96.42) (width 0.1524) (layer B.Cu) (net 14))
 (segment (start 114.9379 93.468) (end 114.9379 95.3579) (width 0.1524) (layer B.Cu) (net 14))
 (segment (start 115.9852 92.4207) (end 114.9379 93.468) (width 0.1524) (layer B.Cu) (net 14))
 (segment (start 108.875 94) (end 108.875 92.9711) (width 0.1524) (layer F.Cu) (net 14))
 (segment (start 114.1566 92.0366) (end 116 93.88) (width 0.1524) (layer F.Cu) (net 15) (status 800000))
 (segment (start 110.4595 92.0366) (end 114.1566 92.0366) (width 0.1524) (layer F.Cu) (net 15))
 (segment (start 109.525 92.9711) (end 110.4595 92.0366) (width 0.1524) (layer F.Cu) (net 15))
 (segment (start 109.525 94) (end 109.525 92.9711) (width 0.1524) (layer F.Cu) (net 15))
 (segment (start 102.9251 92.22) (end 106.105 92.22) (width 0.1524) (layer F.Cu) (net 5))
 (segment (start 106.35 92.475) (end 106.3485 92.475) (width 0.1524) (layer F.Cu) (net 5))
 (segment (start 106.3485 92.4735) (end 106.35 92.475) (width 0.1524) (layer F.Cu) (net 5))
 (segment (start 106.3485 92.4635) (end 106.3485 92.4735) (width 0.1524) (layer F.Cu) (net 5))
 (segment (start 106.105 92.22) (end 106.3485 92.4635) (width 0.1524) (layer F.Cu) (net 5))
 (via (at 102.9251 92.22) (size 0.6096) (layers F.Cu B.Cu) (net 5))
 (segment (start 106.3485 94.5387) (end 106.3485 92.475) (width 0.1524) (layer F.Cu) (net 5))
 (segment (start 111.475 94) (end 111.475 95.0289) (width 0.1524) (layer F.Cu) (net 5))
 (segment (start 111.475 95.0289) (end 109.6401 96.8638) (width 0.1524) (layer F.Cu) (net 5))
 (segment (start 109.6401 96.8638) (end 108.6736 96.8638) (width 0.1524) (layer F.Cu) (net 5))
 (segment (start 108.6736 96.8638) (end 106.3485 94.5387) (width 0.1524) (layer F.Cu) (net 5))
 (segment (start 101.939 92.216) (end 102.6251 92.216) (width 0.1524) (layer B.Cu) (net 5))
 (segment (start 102.6291 92.22) (end 102.9251 92.22) (width 0.1524) (layer B.Cu) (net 5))
 (segment (start 102.6251 92.216) (end 102.6291 92.22) (width 0.1524) (layer B.Cu) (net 5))
 (segment (start 103.145 92.22) (end 103.225 92.3) (width 0.1524) (layer B.Cu) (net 5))
 (segment (start 102.9251 92.22) (end 103.145 92.22) (width 0.1524) (layer B.Cu) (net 5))
 (segment (start 104 92.3) (end 103.225 92.3) (width 0.1524) (layer B.Cu) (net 5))
 (via (at 112.7498 95.8586) (size 0.6096) (layers F.Cu B.Cu) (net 12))
 (segment (start 110.865 94.5) (end 110.865 93.2711) (width 0.1524) (layer B.Cu) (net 12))
 (segment (start 112.7497 95.8586) (end 112.7498 95.8586) (width 0.1524) (layer B.Cu) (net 12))
 (segment (start 112.7497 93.4511) (end 112.7497 95.8586) (width 0.1524) (layer B.Cu) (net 12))
 (segment (start 112.5697 93.2711) (end 112.7497 93.4511) (width 0.1524) (layer B.Cu) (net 12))
 (segment (start 110.865 93.2711) (end 112.5697 93.2711) (width 0.1524) (layer B.Cu) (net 12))
 (segment (start 113.425 95.1834) (end 112.7498 95.8586) (width 0.1524) (layer F.Cu) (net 12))
 (segment (start 113.425 94) (end 113.425 95.1834) (width 0.1524) (layer F.Cu) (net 12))
 (via (at 111.9802 97.8489) (size 0.6096) (layers F.Cu B.Cu) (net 10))
 (segment (start 111.9802 95.8237) (end 111.9802 97.8489) (width 0.1524) (layer F.Cu) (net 10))
 (segment (start 112.775 95.0289) (end 111.9802 95.8237) (width 0.1524) (layer F.Cu) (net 10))
 (segment (start 112.135 98.0037) (end 112.135 101.5) (width 0.1524) (layer B.Cu) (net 10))
 (segment (start 111.9802 97.8489) (end 112.135 98.0037) (width 0.1524) (layer B.Cu) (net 10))
 (segment (start 112.775 94) (end 112.775 95.0289) (width 0.1524) (layer F.Cu) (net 10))
 (via (at 111.1262 96.3061) (size 0.6096) (layers F.Cu B.Cu) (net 11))
 (segment (start 110.1721 96.306) (end 109.595 95.7289) (width 0.1524) (layer B.Cu) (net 11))
 (segment (start 111.1262 96.306) (end 110.1721 96.306) (width 0.1524) (layer B.Cu) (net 11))
 (segment (start 111.1262 96.3061) (end 111.1262 96.306) (width 0.1524) (layer B.Cu) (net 11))
 (segment (start 111.1263 96.3061) (end 111.1262 96.3061) (width 0.1524) (layer F.Cu) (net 11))
 (segment (start 111.1263 96.0276) (end 111.1263 96.3061) (width 0.1524) (layer F.Cu) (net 11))
 (segment (start 112.125 95.0289) (end 111.1263 96.0276) (width 0.1524) (layer F.Cu) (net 11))
 (segment (start 109.595 94.5) (end 109.595 95.7289) (width 0.1524) (layer B.Cu) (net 11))
 (segment (start 112.125 94) (end 112.125 95.0289) (width 0.1524) (layer F.Cu) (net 11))
 (segment (start 109.525 100) (end 109.525 98.9711) (width 0.1524) (layer F.Cu) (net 8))
 (segment (start 107.2539 96.7) (end 109.525 98.9711) (width 0.1524) (layer F.Cu) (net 8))
 (segment (start 104.925 96.7) (end 107.2539 96.7) (width 0.1524) (layer F.Cu) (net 8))
 (via (at 113.855 97.1001) (size 0.6096) (layers F.Cu B.Cu) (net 16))
 (segment (start 113.855 97.2411) (end 113.855 97.1001) (width 0.1524) (layer F.Cu) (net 16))
 (segment (start 112.125 98.9711) (end 113.855 97.2411) (width 0.1524) (layer F.Cu) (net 16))
 (segment (start 114.6327 91.8673) (end 116.25 90.25) (width 0.1524) (layer B.Cu) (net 16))
 (segment (start 114.6327 96.3224) (end 114.6327 91.8673) (width 0.1524) (layer B.Cu) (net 16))
 (segment (start 113.855 97.1001) (end 114.6327 96.3224) (width 0.1524) (layer B.Cu) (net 16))
 (segment (start 112.125 100) (end 112.125 98.9711) (width 0.1524) (layer F.Cu) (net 16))
 (segment (start 119.5937 91.5937) (end 118.25 90.25) (width 0.1524) (layer F.Cu) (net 17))
 (segment (start 119.5937 94.2763) (end 119.5937 91.5937) (width 0.1524) (layer F.Cu) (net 17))
 (segment (start 118.479 95.391) (end 119.5937 94.2763) (width 0.1524) (layer F.Cu) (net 17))
 (segment (start 115.5146 95.391) (end 118.479 95.391) (width 0.1524) (layer F.Cu) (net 17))
 (segment (start 114.8239 96.0817) (end 115.5146 95.391) (width 0.1524) (layer F.Cu) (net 17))
 (segment (start 114.8239 96.8861) (end 114.8239 96.0817) (width 0.1524) (layer F.Cu) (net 17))
 (segment (start 112.775 98.935) (end 114.8239 96.8861) (width 0.1524) (layer F.Cu) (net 17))
 (segment (start 112.775 100) (end 112.775 98.935) (width 0.1524) (layer F.Cu) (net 17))
 (via (at 108.4563 102.5105) (size 0.6096) (layers F.Cu B.Cu) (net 9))
 (segment (start 108.225 100) (end 108.225 101.0289) (width 0.1524) (layer F.Cu) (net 9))
 (segment (start 106.1 102) (end 106.875 102) (width 0.1524) (layer F.Cu) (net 9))
 (segment (start 108.6747 102.7289) (end 113.405 102.7289) (width 0.1524) (layer B.Cu) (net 9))
 (segment (start 108.4563 102.5105) (end 108.6747 102.7289) (width 0.1524) (layer B.Cu) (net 9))
 (segment (start 113.405 101.5) (end 113.405 102.7289) (width 0.1524) (layer B.Cu) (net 9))
 (segment (start 106.8918 101.9832) (end 107.929 101.9832) (width 0.1524) (layer F.Cu) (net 9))
 (segment (start 106.875 102) (end 106.8918 101.9832) (width 0.1524) (layer F.Cu) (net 9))
 (segment (start 108.2415 101.6707) (end 107.929 101.9832) (width 0.1524) (layer F.Cu) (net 9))
 (segment (start 108.2415 101.0454) (end 108.2415 101.6707) (width 0.1524) (layer F.Cu) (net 9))
 (segment (start 108.225 101.0289) (end 108.2415 101.0454) (width 0.1524) (layer F.Cu) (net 9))
 (segment (start 107.929 101.9832) (end 108.4563 102.5105) (width 0.1524) (layer F.Cu) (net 9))
 (segment (start 114.6 100.338) (end 114.562 100.338) (width 0.1524) (layer F.Cu) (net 18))
 (segment (start 110.825 101.35) (end 110.825 100) (width 0.1524) (layer F.Cu) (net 18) (status 800000))
 (segment (start 110.85 101.375) (end 110.825 101.35) (width 0.1524) (layer F.Cu) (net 18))
 (segment (start 113.525 101.375) (end 110.85 101.375) (width 0.1524) (layer F.Cu) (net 18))
 (segment (start 114.562 100.338) (end 113.525 101.375) (width 0.1524) (layer F.Cu) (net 18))
 (segment (start 117.122 100.338) (end 118.5 98.96) (width 0.1524) (layer F.Cu) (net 18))
 (segment (start 114.6 100.338) (end 117.122 100.338) (width 0.1524) (layer F.Cu) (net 18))
 (segment (start 118.6711 99.1311) (end 118.6711 99.225) (width 0.1524) (layer B.Cu) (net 18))
 (segment (start 118.5 98.96) (end 118.6711 99.1311) (width 0.1524) (layer B.Cu) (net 18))
 (segment (start 119.3 99.225) (end 118.6711 99.225) (width 0.1524) (layer B.Cu) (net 18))
 (segment (start 113.425 100) (end 113.425 98.9711) (width 0.1524) (layer F.Cu) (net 20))
 (segment (start 117.23 97.69) (end 118.5 96.42) (width 0.1524) (layer F.Cu) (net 20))
 (segment (start 114.7061 97.69) (end 117.23 97.69) (width 0.1524) (layer F.Cu) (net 20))
 (segment (start 113.425 98.9711) (end 114.7061 97.69) (width 0.1524) (layer F.Cu) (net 20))
 (via (at 107.0978 97.8009) (size 0.6096) (layers F.Cu B.Cu) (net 13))
 (segment (start 108.268 98.9711) (end 107.0978 97.8009) (width 0.1524) (layer F.Cu) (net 13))
 (segment (start 108.875 98.9711) (end 108.268 98.9711) (width 0.1524) (layer F.Cu) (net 13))
 (segment (start 112.135 94.5) (end 112.135 95.7289) (width 0.1524) (layer B.Cu) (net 13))
 (segment (start 108.875 100) (end 108.875 98.9711) (width 0.1524) (layer F.Cu) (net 13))
 (segment (start 112.135 96.1338) (end 112.135 95.7289) (width 0.1524) (layer B.Cu) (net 13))
 (segment (start 110.4679 97.8009) (end 112.135 96.1338) (width 0.1524) (layer B.Cu) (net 13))
 (segment (start 107.0978 97.8009) (end 110.4679 97.8009) (width 0.1524) (layer B.Cu) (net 13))
 (segment (start 117.451 94.929) (end 118.5 93.88) (width 0.1524) (layer F.Cu) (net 19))
 (segment (start 115.1737 94.929) (end 117.451 94.929) (width 0.1524) (layer F.Cu) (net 19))
 (segment (start 112.5139 97.5888) (end 115.1737 94.929) (width 0.1524) (layer F.Cu) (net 19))
 (segment (start 112.5139 98.0701) (end 112.5139 97.5888) (width 0.1524) (layer F.Cu) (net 19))
 (segment (start 111.6129 98.9711) (end 112.5139 98.0701) (width 0.1524) (layer F.Cu) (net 19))
 (segment (start 111.475 98.9711) (end 111.6129 98.9711) (width 0.1524) (layer F.Cu) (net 19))
 (segment (start 111.475 100) (end 111.475 98.9711) (width 0.1524) (layer F.Cu) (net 19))
 (segment (start 98.5303 101.54) (end 98.5703 101.5) (width 0.254) (layer B.Cu) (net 4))
 (segment (start 97.5 101.54) (end 98.5303 101.54) (width 0.254) (layer B.Cu) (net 4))
 (segment (start 99.45 101.5) (end 98.5703 101.5) (width 0.254) (layer B.Cu) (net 4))
 (segment (start 100.025 100.1453) (end 99.45 100.7203) (width 0.254) (layer B.Cu) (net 4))
 (segment (start 100.025 99.175) (end 100.025 100.1453) (width 0.254) (layer B.Cu) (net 4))
 (segment (start 99.45 101.5) (end 99.45 100.7203) (width 0.254) (layer B.Cu) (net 4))
 (segment (start 97.5 90.5) (end 100.0479 90.5) (width 0.254) (layer B.Cu) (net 21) (status 400000))
 (segment (start 100.0479 90.5) (end 100.3639 90.184) (width 0.254) (layer B.Cu) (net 21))
 (segment (start 100.3639 90.184) (end 101.05 90.184) (width 0.254) (layer B.Cu) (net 21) (status 800000))
 (segment (start 100.0479 90.5) (end 100.3639 90.184) (width 0.1524) (layer B.Cu) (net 21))
 (segment (start 101.05 90.184) (end 100.3639 90.184) (width 0.1524) (layer B.Cu) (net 21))
 (segment (start 97.5 93.5703) (end 97.5 93.04) (width 0.254) (layer B.Cu) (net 22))
 (segment (start 100.025 96.0953) (end 97.5 93.5703) (width 0.254) (layer B.Cu) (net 22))
 (segment (start 100.025 96.875) (end 100.025 96.0953) (width 0.254) (layer B.Cu) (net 22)))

